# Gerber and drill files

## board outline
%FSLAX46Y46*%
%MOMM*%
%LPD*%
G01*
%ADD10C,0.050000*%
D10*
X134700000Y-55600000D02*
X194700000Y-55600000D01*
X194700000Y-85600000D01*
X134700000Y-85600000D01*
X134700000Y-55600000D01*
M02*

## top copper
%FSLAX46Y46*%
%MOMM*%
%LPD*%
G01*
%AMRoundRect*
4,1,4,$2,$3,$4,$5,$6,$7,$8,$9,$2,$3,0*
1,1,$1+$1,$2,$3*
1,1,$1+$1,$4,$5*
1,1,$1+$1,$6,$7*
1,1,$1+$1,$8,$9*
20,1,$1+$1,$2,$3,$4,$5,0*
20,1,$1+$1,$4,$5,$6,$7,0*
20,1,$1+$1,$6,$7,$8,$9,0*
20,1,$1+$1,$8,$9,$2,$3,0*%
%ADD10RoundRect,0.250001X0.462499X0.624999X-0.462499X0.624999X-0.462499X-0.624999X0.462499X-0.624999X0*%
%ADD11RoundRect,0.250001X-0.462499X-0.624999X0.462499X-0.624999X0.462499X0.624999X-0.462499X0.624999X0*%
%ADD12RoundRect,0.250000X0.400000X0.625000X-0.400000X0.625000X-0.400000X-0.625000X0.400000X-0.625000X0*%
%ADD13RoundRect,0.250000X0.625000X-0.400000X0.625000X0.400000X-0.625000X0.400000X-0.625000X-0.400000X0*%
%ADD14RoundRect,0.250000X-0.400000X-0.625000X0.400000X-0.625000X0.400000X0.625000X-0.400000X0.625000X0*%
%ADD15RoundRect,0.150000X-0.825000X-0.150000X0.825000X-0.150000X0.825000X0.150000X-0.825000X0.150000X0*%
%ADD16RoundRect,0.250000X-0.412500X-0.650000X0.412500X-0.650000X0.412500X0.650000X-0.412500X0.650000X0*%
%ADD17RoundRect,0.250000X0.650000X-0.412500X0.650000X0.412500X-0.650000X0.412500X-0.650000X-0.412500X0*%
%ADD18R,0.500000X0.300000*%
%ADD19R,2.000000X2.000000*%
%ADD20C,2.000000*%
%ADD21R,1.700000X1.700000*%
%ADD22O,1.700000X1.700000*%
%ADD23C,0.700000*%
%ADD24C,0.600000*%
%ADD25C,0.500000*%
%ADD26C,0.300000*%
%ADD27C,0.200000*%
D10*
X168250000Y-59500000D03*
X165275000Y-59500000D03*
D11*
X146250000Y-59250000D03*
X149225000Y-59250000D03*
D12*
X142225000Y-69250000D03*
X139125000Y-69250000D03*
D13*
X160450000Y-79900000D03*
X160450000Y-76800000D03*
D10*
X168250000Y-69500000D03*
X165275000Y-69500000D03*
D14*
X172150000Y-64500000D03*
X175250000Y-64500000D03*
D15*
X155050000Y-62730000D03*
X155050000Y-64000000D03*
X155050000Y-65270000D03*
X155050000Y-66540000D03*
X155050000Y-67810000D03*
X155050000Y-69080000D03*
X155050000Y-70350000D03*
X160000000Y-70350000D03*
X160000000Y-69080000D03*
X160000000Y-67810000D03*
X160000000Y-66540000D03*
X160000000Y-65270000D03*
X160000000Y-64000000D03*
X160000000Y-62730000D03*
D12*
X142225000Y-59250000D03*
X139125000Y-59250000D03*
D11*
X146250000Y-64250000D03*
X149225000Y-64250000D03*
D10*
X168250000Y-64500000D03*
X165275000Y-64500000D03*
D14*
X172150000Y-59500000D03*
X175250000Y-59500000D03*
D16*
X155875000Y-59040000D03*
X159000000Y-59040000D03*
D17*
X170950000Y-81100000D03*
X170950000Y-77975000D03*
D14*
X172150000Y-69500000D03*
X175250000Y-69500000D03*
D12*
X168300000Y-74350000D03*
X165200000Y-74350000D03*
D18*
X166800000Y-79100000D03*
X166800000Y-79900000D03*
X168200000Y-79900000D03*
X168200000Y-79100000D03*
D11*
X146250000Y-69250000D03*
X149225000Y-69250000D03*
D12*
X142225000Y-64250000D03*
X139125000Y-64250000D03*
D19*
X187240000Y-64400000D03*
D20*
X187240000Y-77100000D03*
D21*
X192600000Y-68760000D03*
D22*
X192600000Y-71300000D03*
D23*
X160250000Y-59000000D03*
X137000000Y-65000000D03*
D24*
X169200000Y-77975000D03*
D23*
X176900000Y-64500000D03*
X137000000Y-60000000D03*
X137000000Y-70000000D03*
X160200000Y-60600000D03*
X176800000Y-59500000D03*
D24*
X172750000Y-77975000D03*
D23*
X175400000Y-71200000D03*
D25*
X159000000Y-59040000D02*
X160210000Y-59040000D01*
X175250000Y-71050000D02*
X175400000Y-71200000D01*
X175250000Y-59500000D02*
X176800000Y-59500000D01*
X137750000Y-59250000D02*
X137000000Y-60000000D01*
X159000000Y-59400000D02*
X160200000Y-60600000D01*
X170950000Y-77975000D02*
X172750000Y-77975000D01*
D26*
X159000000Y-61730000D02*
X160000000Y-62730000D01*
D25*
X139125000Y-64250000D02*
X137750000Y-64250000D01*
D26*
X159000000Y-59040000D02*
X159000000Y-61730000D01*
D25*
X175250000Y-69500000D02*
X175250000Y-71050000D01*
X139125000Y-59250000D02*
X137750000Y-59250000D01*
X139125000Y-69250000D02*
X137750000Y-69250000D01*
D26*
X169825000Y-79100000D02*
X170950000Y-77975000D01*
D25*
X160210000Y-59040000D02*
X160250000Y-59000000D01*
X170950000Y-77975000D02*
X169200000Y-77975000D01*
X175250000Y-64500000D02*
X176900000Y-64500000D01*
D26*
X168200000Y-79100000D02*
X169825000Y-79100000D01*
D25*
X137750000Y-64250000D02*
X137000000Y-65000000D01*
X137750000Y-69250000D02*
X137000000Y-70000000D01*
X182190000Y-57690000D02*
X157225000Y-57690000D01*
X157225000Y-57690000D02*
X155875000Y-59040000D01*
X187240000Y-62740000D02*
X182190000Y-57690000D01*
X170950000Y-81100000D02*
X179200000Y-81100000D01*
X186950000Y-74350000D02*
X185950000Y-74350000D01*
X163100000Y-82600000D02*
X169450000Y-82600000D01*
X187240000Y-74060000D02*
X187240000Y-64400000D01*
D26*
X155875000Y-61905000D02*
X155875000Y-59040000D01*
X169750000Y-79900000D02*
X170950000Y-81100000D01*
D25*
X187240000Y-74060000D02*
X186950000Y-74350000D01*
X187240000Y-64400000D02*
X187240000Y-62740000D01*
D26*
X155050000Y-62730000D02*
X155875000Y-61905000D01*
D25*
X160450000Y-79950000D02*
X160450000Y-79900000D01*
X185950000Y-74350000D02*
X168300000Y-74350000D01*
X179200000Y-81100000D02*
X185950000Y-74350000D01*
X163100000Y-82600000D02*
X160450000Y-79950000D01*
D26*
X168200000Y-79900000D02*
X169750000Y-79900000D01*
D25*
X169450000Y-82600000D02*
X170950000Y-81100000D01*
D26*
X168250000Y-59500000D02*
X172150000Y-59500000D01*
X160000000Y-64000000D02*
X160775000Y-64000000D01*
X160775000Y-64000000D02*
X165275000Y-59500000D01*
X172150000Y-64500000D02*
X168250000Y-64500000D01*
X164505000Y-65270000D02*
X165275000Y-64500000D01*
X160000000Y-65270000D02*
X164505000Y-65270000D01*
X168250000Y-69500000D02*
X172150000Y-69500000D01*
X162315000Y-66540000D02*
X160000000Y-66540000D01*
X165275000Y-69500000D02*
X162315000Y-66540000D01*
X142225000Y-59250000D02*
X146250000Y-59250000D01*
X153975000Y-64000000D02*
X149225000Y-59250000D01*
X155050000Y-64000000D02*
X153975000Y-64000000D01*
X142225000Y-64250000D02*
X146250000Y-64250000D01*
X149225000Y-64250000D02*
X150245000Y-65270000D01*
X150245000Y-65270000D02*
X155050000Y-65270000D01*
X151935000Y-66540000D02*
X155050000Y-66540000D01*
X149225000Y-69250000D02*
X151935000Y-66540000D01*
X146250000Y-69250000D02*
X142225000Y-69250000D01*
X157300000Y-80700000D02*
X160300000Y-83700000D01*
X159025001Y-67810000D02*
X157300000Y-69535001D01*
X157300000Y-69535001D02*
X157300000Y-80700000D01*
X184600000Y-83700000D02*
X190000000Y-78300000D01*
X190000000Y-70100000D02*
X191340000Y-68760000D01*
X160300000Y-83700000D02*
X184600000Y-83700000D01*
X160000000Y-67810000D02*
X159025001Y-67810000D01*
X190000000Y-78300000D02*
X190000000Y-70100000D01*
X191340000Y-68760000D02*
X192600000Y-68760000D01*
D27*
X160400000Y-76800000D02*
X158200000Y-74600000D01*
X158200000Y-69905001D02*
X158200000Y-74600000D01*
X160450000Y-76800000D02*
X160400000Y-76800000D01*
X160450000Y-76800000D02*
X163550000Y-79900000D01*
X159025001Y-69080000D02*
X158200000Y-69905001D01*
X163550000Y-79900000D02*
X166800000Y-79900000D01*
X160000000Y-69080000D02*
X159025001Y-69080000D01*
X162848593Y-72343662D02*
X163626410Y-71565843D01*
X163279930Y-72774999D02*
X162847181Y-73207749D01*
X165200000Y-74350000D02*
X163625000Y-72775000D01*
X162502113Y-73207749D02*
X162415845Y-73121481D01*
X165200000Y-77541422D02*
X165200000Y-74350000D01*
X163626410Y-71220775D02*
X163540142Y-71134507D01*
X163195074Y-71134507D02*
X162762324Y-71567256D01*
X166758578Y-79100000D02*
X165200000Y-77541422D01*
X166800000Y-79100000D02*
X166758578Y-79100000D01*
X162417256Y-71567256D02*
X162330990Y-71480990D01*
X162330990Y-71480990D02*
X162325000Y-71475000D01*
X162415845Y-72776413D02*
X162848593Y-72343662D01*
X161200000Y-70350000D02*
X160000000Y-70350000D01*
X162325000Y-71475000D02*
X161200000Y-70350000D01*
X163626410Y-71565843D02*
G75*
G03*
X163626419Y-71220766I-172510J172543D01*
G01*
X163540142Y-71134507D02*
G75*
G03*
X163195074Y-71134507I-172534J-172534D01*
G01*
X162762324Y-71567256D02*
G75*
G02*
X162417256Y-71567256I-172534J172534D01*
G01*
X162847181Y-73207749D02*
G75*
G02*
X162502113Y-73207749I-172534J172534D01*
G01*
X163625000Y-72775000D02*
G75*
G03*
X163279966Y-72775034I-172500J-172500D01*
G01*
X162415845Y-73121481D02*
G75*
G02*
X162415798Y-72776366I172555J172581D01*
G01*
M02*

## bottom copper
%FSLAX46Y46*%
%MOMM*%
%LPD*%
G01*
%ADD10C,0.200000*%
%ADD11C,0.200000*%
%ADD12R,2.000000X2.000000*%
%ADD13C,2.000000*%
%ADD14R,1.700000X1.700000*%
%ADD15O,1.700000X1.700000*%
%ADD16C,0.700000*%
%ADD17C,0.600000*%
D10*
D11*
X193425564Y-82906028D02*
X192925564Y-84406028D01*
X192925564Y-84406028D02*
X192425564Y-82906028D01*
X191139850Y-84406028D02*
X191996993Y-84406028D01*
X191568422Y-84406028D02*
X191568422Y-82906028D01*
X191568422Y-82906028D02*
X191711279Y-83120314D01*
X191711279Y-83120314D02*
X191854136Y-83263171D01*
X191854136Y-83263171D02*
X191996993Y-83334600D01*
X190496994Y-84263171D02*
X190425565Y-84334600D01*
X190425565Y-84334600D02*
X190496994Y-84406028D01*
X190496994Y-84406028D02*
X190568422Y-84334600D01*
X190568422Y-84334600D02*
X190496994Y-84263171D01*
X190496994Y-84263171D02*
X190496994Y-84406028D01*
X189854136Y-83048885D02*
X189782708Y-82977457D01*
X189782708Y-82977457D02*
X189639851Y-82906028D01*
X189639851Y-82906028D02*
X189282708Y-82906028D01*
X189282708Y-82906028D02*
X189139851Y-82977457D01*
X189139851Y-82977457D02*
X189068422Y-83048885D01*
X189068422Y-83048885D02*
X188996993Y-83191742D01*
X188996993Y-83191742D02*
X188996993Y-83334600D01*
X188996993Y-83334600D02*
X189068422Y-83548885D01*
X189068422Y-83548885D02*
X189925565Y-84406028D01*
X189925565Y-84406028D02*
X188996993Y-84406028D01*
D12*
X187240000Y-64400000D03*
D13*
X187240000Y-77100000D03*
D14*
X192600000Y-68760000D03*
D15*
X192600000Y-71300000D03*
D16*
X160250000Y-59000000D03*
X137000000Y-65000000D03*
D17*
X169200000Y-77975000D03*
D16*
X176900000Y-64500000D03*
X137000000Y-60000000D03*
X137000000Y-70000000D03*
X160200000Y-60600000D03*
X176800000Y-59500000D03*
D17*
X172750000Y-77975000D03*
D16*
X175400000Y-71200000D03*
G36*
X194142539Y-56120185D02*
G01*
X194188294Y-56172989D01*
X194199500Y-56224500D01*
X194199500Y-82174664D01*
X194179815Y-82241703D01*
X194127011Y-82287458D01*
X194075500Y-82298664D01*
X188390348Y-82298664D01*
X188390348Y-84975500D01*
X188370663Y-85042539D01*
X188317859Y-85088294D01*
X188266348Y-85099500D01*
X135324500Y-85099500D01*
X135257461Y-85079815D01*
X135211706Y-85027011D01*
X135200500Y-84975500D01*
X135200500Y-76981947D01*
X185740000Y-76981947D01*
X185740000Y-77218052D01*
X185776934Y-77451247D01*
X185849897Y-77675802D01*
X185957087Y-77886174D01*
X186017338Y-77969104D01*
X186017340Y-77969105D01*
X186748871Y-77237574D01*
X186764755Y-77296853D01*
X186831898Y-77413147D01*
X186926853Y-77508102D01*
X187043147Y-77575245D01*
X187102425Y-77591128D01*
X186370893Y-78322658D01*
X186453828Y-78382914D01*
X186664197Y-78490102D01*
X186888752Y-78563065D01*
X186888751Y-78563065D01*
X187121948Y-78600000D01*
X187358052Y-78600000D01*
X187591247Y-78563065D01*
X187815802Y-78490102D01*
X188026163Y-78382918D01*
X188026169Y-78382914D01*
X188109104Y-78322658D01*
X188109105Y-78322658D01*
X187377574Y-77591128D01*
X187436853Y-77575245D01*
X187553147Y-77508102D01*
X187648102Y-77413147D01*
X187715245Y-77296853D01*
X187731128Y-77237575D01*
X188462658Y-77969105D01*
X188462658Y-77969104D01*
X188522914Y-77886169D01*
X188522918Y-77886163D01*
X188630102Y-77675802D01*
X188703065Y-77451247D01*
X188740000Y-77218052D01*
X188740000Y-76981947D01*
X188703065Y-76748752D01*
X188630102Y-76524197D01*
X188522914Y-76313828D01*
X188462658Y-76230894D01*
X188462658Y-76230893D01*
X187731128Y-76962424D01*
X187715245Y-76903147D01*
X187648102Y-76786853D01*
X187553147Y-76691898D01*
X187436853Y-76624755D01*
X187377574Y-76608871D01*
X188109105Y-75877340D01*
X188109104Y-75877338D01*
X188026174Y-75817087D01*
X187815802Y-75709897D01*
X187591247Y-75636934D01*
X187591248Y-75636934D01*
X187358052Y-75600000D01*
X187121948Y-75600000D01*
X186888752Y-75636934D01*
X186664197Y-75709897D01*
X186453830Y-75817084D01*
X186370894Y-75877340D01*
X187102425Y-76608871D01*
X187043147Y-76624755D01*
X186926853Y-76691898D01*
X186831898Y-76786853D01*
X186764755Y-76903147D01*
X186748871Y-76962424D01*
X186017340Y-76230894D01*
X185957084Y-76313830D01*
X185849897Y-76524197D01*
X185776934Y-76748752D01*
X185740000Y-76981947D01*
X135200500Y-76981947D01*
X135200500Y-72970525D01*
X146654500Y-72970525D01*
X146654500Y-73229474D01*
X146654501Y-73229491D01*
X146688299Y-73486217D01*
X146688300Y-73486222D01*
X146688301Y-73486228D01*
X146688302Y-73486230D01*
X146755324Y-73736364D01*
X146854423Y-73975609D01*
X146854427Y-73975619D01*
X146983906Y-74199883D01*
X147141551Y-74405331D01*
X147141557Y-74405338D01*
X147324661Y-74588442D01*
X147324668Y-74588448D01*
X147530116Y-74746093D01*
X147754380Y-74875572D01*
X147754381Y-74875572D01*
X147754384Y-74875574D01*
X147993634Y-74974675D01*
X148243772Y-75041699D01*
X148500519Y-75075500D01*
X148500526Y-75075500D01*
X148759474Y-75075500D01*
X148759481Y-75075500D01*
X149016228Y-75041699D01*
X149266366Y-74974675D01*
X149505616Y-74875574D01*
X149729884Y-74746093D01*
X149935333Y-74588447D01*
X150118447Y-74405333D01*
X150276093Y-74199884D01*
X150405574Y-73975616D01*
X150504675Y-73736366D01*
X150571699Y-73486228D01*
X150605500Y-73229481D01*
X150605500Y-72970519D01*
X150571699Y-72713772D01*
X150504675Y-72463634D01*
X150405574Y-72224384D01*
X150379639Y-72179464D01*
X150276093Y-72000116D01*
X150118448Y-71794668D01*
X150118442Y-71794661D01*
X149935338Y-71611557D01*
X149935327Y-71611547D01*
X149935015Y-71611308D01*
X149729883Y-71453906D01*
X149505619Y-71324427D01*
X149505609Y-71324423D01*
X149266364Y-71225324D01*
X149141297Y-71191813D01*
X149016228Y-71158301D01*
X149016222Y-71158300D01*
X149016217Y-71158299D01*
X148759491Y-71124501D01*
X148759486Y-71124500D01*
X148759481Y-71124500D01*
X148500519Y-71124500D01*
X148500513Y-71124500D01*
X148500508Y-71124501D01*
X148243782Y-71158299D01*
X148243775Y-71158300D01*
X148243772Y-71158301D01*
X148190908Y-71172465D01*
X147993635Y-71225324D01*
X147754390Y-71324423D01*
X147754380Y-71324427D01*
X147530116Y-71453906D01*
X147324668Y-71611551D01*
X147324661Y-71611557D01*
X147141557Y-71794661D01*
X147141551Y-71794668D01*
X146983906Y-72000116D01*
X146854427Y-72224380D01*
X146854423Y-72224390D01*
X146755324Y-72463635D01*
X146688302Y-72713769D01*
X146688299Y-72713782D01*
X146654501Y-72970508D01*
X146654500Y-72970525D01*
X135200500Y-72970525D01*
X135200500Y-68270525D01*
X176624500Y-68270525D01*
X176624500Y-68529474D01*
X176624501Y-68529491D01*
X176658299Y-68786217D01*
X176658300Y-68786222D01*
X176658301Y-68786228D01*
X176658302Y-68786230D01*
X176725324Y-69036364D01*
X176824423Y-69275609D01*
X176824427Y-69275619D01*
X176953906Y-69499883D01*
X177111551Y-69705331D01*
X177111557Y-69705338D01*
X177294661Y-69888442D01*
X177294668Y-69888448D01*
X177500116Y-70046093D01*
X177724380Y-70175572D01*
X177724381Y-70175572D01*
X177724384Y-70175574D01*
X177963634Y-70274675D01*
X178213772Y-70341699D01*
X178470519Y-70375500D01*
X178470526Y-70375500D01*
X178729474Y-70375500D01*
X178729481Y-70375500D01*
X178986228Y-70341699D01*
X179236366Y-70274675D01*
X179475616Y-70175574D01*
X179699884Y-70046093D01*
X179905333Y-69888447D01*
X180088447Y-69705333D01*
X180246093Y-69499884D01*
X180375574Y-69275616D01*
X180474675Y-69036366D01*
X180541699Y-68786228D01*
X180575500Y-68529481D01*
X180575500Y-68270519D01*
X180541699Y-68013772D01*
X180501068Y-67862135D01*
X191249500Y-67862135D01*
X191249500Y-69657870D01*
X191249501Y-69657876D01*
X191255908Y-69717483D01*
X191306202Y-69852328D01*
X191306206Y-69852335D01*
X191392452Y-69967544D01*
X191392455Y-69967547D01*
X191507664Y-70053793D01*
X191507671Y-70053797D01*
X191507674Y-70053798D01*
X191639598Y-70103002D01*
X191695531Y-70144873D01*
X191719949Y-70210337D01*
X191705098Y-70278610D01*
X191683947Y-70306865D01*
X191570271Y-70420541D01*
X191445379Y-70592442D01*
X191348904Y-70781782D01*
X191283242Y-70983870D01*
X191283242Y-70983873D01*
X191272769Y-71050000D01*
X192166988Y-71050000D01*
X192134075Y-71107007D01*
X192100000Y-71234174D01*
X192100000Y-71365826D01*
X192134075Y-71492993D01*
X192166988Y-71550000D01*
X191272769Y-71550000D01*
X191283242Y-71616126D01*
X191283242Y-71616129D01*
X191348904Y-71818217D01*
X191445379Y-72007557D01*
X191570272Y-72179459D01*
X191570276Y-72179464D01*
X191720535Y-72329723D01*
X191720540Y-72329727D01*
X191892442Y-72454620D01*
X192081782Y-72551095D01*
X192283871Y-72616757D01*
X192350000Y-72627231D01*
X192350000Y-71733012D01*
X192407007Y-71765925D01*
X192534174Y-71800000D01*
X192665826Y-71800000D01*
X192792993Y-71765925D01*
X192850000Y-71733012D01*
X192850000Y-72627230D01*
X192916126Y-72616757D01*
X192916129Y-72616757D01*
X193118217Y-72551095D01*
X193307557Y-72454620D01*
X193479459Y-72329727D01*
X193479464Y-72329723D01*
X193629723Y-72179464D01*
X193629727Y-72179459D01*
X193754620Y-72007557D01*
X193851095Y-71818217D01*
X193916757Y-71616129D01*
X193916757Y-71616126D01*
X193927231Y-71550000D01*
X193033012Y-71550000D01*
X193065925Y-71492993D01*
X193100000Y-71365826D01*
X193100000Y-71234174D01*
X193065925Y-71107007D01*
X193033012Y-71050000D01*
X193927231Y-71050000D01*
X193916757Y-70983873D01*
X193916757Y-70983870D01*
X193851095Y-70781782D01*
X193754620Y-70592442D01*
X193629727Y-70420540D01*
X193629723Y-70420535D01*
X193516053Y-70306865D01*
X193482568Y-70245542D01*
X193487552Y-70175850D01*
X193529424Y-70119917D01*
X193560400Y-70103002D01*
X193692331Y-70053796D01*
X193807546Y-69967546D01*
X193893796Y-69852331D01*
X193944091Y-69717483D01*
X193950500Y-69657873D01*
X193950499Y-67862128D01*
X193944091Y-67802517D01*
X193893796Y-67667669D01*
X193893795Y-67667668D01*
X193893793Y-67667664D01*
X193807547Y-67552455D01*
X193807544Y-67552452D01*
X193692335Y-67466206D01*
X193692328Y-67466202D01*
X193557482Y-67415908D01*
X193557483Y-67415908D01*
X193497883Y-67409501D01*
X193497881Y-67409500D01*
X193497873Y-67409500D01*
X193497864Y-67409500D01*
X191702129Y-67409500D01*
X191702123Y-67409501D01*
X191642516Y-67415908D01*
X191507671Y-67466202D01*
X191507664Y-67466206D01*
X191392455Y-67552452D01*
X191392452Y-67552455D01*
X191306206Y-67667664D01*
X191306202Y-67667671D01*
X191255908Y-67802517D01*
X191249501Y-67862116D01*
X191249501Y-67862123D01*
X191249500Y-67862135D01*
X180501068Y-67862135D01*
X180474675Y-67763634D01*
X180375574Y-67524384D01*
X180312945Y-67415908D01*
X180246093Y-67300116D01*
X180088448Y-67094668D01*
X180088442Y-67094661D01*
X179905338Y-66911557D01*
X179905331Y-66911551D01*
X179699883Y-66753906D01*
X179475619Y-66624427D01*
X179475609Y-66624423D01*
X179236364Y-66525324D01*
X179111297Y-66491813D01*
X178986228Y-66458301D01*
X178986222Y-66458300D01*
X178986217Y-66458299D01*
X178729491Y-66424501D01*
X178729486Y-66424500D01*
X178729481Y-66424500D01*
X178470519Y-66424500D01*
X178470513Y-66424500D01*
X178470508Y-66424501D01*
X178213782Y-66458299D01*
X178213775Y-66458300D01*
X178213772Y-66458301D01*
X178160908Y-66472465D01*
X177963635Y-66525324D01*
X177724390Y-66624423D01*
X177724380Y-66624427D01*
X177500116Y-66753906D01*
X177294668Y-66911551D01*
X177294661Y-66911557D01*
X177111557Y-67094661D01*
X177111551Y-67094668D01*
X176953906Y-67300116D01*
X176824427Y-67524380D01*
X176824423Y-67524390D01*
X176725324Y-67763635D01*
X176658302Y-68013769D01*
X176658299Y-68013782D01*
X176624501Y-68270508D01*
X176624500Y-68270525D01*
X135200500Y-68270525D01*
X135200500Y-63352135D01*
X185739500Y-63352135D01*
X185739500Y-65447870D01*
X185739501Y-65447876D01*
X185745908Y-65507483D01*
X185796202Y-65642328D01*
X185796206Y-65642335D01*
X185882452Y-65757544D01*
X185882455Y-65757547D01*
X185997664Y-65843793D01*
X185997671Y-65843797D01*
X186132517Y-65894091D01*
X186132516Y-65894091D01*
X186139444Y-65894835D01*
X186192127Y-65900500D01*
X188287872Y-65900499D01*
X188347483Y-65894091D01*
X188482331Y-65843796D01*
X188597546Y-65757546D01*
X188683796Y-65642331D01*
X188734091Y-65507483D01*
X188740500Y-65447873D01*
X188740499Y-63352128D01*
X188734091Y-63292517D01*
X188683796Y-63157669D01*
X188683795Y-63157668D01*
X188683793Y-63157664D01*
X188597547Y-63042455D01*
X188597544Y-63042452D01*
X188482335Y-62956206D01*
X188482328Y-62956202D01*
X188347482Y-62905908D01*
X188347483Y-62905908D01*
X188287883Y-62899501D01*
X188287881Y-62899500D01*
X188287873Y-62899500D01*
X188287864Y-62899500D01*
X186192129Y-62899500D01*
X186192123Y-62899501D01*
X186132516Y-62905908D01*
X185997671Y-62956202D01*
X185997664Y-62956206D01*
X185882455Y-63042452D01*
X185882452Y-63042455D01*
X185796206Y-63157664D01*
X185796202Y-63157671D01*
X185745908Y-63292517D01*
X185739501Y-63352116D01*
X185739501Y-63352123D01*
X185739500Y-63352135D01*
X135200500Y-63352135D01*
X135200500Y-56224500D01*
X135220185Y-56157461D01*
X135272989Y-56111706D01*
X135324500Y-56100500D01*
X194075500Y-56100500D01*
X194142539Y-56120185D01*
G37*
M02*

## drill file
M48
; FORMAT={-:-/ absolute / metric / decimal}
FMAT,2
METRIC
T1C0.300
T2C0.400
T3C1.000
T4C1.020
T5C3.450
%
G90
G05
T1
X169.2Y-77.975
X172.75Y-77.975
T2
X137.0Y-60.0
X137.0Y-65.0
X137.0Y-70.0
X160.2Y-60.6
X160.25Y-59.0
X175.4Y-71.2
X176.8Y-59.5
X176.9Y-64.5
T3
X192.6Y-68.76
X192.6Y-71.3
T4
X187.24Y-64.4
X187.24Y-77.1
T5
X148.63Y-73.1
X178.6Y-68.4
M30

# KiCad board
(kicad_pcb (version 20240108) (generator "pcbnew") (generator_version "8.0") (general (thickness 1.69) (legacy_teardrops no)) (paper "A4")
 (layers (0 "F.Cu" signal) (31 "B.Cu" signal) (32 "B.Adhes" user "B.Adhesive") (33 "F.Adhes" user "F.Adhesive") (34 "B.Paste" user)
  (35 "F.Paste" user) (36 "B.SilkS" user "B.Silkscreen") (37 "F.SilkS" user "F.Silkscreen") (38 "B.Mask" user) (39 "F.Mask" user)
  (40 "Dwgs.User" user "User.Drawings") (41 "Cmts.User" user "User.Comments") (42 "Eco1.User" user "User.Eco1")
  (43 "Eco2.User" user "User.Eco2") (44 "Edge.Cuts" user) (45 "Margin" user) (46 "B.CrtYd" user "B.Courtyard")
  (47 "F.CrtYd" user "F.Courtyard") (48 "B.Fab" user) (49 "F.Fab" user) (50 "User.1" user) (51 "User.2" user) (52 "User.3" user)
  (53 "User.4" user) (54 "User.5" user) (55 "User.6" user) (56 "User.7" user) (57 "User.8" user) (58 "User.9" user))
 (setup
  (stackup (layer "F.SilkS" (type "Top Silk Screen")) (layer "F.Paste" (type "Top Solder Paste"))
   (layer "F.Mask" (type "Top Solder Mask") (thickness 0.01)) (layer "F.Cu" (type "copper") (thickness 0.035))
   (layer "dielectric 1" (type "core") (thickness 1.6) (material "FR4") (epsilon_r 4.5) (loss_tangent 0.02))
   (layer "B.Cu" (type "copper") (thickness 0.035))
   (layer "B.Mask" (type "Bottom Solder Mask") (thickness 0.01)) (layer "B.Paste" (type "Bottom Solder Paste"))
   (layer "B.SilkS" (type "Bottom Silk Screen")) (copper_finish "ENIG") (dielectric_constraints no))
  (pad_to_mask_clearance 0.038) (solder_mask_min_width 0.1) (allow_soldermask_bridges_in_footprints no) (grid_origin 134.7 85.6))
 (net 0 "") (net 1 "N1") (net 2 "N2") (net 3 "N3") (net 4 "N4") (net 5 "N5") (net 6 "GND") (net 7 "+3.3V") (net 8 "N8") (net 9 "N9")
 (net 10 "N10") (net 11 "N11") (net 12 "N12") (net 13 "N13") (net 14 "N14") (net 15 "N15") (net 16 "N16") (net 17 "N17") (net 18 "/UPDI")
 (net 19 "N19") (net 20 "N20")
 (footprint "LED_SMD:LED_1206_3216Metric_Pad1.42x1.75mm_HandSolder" (layer "F.Cu") (at 166.7625 59.5 180)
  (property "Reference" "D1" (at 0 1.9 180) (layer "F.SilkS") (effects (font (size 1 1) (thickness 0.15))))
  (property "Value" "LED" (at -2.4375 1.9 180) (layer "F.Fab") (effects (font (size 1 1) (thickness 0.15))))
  (pad "1" smd roundrect (at -1.4875 0 180) (size 1.425 1.75) (layers "F.Cu" "F.Paste" "F.Mask") (roundrect_rratio 0.175439) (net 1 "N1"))
  (pad "2" smd roundrect (at 1.4875 0 180) (size 1.425 1.75) (layers "F.Cu" "F.Paste" "F.Mask") (roundrect_rratio 0.175439) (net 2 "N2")))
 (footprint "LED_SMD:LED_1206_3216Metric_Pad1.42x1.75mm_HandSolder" (layer "F.Cu") (at 147.7375 59.25)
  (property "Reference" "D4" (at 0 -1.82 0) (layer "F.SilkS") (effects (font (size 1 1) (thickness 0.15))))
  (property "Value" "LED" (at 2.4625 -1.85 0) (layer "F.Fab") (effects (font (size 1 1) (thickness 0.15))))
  (pad "1" smd roundrect (at -1.4875 0) (size 1.425 1.75) (layers "F.Cu" "F.Paste" "F.Mask") (roundrect_rratio 0.175439) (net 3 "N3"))
  (pad "2" smd roundrect (at 1.4875 0) (size 1.425 1.75) (layers "F.Cu" "F.Paste" "F.Mask") (roundrect_rratio 0.175439) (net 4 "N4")))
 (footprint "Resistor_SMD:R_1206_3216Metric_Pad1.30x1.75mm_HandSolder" (layer "F.Cu") (at 140.675 69.25 180)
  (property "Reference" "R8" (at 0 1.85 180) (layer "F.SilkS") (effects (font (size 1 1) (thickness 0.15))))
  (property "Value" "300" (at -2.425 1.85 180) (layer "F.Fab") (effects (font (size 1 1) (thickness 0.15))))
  (pad "1" smd roundrect (at -1.55 0 180) (size 1.3 1.75) (layers "F.Cu" "F.Paste" "F.Mask") (roundrect_rratio 0.192308) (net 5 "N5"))
  (pad "2" smd roundrect (at 1.55 0 180) (size 1.3 1.75) (layers "F.Cu" "F.Paste" "F.Mask") (roundrect_rratio 0.192308) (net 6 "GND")))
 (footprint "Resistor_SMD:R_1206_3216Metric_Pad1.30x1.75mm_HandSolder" (layer "F.Cu") (at 160.45 78.35 90)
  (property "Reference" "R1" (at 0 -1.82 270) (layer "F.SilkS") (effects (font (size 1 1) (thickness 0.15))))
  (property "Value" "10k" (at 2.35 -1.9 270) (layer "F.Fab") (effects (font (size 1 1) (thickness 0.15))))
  (pad "1" smd roundrect (at -1.55 0 90) (size 1.3 1.75) (layers "F.Cu" "F.Paste" "F.Mask") (roundrect_rratio 0.192308) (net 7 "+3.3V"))
  (pad "2" smd roundrect (at 1.55 0 90) (size 1.3 1.75) (layers "F.Cu" "F.Paste" "F.Mask") (roundrect_rratio 0.192308) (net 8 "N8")))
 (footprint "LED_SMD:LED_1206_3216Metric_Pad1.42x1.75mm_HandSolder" (layer "F.Cu") (at 166.7625 69.5 180)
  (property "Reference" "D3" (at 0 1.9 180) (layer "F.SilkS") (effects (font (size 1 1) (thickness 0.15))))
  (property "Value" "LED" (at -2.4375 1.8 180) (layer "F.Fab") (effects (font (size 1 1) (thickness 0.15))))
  (pad "1" smd roundrect (at -1.4875 0 180) (size 1.425 1.75) (layers "F.Cu" "F.Paste" "F.Mask") (roundrect_rratio 0.175439) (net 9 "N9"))
  (pad "2" smd roundrect (at 1.4875 0 180) (size 1.425 1.75) (layers "F.Cu" "F.Paste" "F.Mask") (roundrect_rratio 0.175439) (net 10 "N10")))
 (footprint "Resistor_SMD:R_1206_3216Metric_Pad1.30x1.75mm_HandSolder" (layer "F.Cu") (at 173.7 64.5)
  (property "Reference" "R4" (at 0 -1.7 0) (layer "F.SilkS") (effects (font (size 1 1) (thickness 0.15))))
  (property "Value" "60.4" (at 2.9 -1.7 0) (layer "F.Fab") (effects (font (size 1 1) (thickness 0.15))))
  (pad "1" smd roundrect (at -1.55 0) (size 1.3 1.75) (layers "F.Cu" "F.Paste" "F.Mask") (roundrect_rratio 0.192308) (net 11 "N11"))
  (pad "2" smd roundrect (at 1.55 0) (size 1.3 1.75) (layers "F.Cu" "F.Paste" "F.Mask") (roundrect_rratio 0.192308) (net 6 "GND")))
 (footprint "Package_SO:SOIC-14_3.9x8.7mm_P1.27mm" (layer "F.Cu") (at 157.525 66.54)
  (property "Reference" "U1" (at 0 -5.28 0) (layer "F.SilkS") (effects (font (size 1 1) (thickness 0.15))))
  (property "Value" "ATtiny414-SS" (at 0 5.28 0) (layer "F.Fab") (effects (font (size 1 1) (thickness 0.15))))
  (pad "1" smd roundrect (at -2.475 -3.81) (size 1.95 0.6) (layers "F.Cu" "F.Paste" "F.Mask") (roundrect_rratio 0.25) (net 7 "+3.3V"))
  (pad "2" smd roundrect (at -2.475 -2.54) (size 1.95 0.6) (layers "F.Cu" "F.Paste" "F.Mask") (roundrect_rratio 0.25) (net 4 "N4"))
  (pad "3" smd roundrect (at -2.475 -1.27) (size 1.95 0.6) (layers "F.Cu" "F.Paste" "F.Mask") (roundrect_rratio 0.25) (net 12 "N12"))
  (pad "4" smd roundrect (at -2.475 0) (size 1.95 0.6) (layers "F.Cu" "F.Paste" "F.Mask") (roundrect_rratio 0.25) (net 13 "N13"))
  (pad "5" smd roundrect (at -2.475 1.27) (size 1.95 0.6) (layers "F.Cu" "F.Paste" "F.Mask") (roundrect_rratio 0.25) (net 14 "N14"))
  (pad "6" smd roundrect (at -2.475 2.54) (size 1.95 0.6) (layers "F.Cu" "F.Paste" "F.Mask") (roundrect_rratio 0.25) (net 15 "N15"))
  (pad "7" smd roundrect (at -2.475 3.81) (size 1.95 0.6) (layers "F.Cu" "F.Paste" "F.Mask") (roundrect_rratio 0.25) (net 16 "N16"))
  (pad "8" smd roundrect (at 2.475 3.81) (size 1.95 0.6) (layers "F.Cu" "F.Paste" "F.Mask") (roundrect_rratio 0.25) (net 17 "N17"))
  (pad "9" smd roundrect (at 2.475 2.54) (size 1.95 0.6) (layers "F.Cu" "F.Paste" "F.Mask") (roundrect_rratio 0.25) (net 8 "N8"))
  (pad "10" smd roundrect (at 2.475 1.27) (size 1.95 0.6) (layers "F.Cu" "F.Paste" "F.Mask") (roundrect_rratio 0.25) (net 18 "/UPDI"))
  (pad "11" smd roundrect (at 2.475 0) (size 1.95 0.6) (layers "F.Cu" "F.Paste" "F.Mask") (roundrect_rratio 0.25) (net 10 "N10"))
  (pad "12" smd roundrect (at 2.475 -1.27) (size 1.95 0.6) (layers "F.Cu" "F.Paste" "F.Mask") (roundrect_rratio 0.25) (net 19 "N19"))
  (pad "13" smd roundrect (at 2.475 -2.54) (size 1.95 0.6) (layers "F.Cu" "F.Paste" "F.Mask") (roundrect_rratio 0.25) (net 2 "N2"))
  (pad "14" smd roundrect (at 2.475 -3.81) (size 1.95 0.6) (layers "F.Cu" "F.Paste" "F.Mask") (roundrect_rratio 0.25) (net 6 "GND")))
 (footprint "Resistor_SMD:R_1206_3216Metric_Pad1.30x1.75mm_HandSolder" (layer "F.Cu") (at 140.675 59.25 180)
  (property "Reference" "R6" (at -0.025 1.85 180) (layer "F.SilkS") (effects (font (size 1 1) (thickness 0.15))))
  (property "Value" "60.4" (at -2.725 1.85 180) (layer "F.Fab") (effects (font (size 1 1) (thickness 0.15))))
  (pad "1" smd roundrect (at -1.55 0 180) (size 1.3 1.75) (layers "F.Cu" "F.Paste" "F.Mask") (roundrect_rratio 0.192308) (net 3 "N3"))
  (pad "2" smd roundrect (at 1.55 0 180) (size 1.3 1.75) (layers "F.Cu" "F.Paste" "F.Mask") (roundrect_rratio 0.192308) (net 6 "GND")))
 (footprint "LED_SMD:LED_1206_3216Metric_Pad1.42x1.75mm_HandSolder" (layer "F.Cu") (at 147.7375 64.25)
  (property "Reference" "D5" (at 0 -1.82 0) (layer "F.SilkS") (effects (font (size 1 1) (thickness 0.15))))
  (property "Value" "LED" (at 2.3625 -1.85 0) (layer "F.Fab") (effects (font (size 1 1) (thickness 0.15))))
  (pad "1" smd roundrect (at -1.4875 0) (size 1.425 1.75) (layers "F.Cu" "F.Paste" "F.Mask") (roundrect_rratio 0.175439) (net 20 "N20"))
  (pad "2" smd roundrect (at 1.4875 0) (size 1.425 1.75) (layers "F.Cu" "F.Paste" "F.Mask") (roundrect_rratio 0.175439) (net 12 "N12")))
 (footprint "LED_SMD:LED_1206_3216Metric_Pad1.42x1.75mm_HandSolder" (layer "F.Cu") (at 166.7625 64.5 180)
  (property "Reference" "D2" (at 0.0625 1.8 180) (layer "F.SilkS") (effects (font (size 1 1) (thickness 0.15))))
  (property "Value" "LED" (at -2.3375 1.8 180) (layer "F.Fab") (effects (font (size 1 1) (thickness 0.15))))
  (pad "1" smd roundrect (at -1.4875 0 180) (size 1.425 1.75) (layers "F.Cu" "F.Paste" "F.Mask") (roundrect_rratio 0.175439) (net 11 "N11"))
  (pad "2" smd roundrect (at 1.4875 0 180) (size 1.425 1.75) (layers "F.Cu" "F.Paste" "F.Mask") (roundrect_rratio 0.175439) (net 19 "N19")))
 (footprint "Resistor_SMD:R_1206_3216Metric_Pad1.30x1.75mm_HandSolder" (layer "F.Cu") (at 173.7 59.5)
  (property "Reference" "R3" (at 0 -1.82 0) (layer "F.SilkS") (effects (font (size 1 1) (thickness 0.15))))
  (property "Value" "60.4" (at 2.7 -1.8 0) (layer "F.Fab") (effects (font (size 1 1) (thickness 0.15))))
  (pad "1" smd roundrect (at -1.55 0) (size 1.3 1.75) (layers "F.Cu" "F.Paste" "F.Mask") (roundrect_rratio 0.192308) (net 1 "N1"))
  (pad "2" smd roundrect (at 1.55 0) (size 1.3 1.75) (layers "F.Cu" "F.Paste" "F.Mask") (roundrect_rratio 0.192308) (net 6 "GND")))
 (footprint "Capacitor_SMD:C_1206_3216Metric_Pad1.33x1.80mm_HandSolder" (layer "F.Cu") (at 157.4375 59.04)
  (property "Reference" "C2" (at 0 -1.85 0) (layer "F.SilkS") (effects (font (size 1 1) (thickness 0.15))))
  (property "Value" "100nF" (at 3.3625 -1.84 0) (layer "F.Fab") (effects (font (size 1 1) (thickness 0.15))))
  (pad "1" smd roundrect (at -1.5625 0) (size 1.325 1.8) (layers "F.Cu" "F.Paste" "F.Mask") (roundrect_rratio 0.188679) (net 7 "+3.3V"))
  (pad "2" smd roundrect (at 1.5625 0) (size 1.325 1.8) (layers "F.Cu" "F.Paste" "F.Mask") (roundrect_rratio 0.188679) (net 6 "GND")))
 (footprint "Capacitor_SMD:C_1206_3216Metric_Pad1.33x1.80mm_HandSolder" (layer "F.Cu") (at 170.95 79.5375 90)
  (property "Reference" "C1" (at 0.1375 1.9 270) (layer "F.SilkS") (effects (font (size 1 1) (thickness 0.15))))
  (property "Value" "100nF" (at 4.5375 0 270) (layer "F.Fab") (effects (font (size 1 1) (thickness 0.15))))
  (pad "1" smd roundrect (at -1.5625 0 90) (size 1.325 1.8) (layers "F.Cu" "F.Paste" "F.Mask") (roundrect_rratio 0.188679) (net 7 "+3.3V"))
  (pad "2" smd roundrect (at 1.5625 0 90) (size 1.325 1.8) (layers "F.Cu" "F.Paste" "F.Mask") (roundrect_rratio 0.188679) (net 6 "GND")))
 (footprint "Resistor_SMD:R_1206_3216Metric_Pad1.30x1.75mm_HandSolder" (layer "F.Cu") (at 173.7 69.5)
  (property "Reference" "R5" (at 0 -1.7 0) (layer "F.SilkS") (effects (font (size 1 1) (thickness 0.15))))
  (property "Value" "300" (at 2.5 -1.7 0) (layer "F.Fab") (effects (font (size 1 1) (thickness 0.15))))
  (pad "1" smd roundrect (at -1.55 0) (size 1.3 1.75) (layers "F.Cu" "F.Paste" "F.Mask") (roundrect_rratio 0.192308) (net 9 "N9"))
  (pad "2" smd roundrect (at 1.55 0) (size 1.3 1.75) (layers "F.Cu" "F.Paste" "F.Mask") (roundrect_rratio 0.192308) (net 6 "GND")))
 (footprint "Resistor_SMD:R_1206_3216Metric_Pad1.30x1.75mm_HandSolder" (layer "F.Cu") (at 166.75 74.35 180)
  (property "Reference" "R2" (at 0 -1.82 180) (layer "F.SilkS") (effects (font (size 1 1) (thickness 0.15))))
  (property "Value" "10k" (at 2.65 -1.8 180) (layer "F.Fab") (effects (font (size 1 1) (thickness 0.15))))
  (pad "1" smd roundrect (at -1.55 0 180) (size 1.3 1.75) (layers "F.Cu" "F.Paste" "F.Mask") (roundrect_rratio 0.192308) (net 7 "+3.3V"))
  (pad "2" smd roundrect (at 1.55 0 180) (size 1.3 1.75) (layers "F.Cu" "F.Paste" "F.Mask") (roundrect_rratio 0.192308) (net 17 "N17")))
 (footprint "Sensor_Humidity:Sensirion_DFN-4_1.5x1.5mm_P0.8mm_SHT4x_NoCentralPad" (layer "F.Cu") (at 167.5 79.5)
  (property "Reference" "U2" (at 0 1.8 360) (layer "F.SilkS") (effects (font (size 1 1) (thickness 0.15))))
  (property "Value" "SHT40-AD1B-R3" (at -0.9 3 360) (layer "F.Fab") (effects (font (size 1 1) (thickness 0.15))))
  (pad "1" smd rect (at -0.7 -0.4) (size 0.5 0.3) (layers "F.Cu" "F.Paste" "F.Mask") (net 17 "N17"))
  (pad "2" smd rect (at -0.7 0.4) (size 0.5 0.3) (layers "F.Cu" "F.Paste" "F.Mask") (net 8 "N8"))
  (pad "3" smd rect (at 0.7 0.4) (size 0.5 0.3) (layers "F.Cu" "F.Paste" "F.Mask") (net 7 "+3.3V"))
  (pad "4" smd rect (at 0.7 -0.4) (size 0.5 0.3) (layers "F.Cu" "F.Paste" "F.Mask") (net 6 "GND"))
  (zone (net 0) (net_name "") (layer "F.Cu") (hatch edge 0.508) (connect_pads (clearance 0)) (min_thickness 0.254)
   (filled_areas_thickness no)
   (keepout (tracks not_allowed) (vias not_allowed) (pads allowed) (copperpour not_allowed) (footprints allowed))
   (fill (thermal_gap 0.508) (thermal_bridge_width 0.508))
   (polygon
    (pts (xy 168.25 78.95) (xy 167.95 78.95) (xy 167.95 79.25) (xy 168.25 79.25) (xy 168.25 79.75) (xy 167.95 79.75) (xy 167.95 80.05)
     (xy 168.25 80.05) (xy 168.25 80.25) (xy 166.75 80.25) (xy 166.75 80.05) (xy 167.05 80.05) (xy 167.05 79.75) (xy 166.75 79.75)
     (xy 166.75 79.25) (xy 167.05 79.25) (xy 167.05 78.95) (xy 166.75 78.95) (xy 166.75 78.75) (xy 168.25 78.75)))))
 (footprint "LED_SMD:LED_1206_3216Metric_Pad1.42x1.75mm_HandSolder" (layer "F.Cu") (at 147.7375 69.25)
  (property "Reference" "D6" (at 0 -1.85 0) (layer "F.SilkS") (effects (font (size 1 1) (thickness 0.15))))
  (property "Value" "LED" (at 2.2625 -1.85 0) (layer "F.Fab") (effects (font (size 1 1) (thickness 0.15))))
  (pad "1" smd roundrect (at -1.4875 0) (size 1.425 1.75) (layers "F.Cu" "F.Paste" "F.Mask") (roundrect_rratio 0.175439) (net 5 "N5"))
  (pad "2" smd roundrect (at 1.4875 0) (size 1.425 1.75) (layers "F.Cu" "F.Paste" "F.Mask") (roundrect_rratio 0.175439) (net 13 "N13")))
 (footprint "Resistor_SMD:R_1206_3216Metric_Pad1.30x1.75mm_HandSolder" (layer "F.Cu") (at 140.675 64.25 180)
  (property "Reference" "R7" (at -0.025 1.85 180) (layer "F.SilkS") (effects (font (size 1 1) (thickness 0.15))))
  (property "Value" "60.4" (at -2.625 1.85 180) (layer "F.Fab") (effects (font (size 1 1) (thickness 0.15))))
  (pad "1" smd roundrect (at -1.55 0 180) (size 1.3 1.75) (layers "F.Cu" "F.Paste" "F.Mask") (roundrect_rratio 0.192308) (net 20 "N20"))
  (pad "2" smd roundrect (at 1.55 0 180) (size 1.3 1.75) (layers "F.Cu" "F.Paste" "F.Mask") (roundrect_rratio 0.192308) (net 6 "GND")))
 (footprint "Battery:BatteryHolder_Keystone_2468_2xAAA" (layer "B.Cu") (at 187.24 64.4 180)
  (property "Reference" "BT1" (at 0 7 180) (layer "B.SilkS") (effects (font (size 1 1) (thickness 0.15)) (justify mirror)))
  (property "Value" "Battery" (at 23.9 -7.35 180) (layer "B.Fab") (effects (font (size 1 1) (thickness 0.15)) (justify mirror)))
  (pad "" np_thru_hole circle (at 8.64 -4 180) (size 3.45 3.45) (drill 3.45) (layers "*.Cu"))
  (pad "" np_thru_hole circle (at 38.61 -8.7 180) (size 3.45 3.45) (drill 3.45) (layers "*.Cu" "*.Mask"))
  (pad "1" thru_hole rect (at 0 0 180) (size 2 2) (drill 1.02) (layers "*.Cu" "*.Mask") (remove_unused_layers no) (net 7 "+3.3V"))
  (pad "2" thru_hole circle (at 0 -12.7 180) (size 2 2) (drill 1.02) (layers "*.Cu" "*.Mask") (remove_unused_layers no) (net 6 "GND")))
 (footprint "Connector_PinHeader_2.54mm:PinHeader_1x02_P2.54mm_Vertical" (layer "B.Cu") (at 192.6 68.76 180)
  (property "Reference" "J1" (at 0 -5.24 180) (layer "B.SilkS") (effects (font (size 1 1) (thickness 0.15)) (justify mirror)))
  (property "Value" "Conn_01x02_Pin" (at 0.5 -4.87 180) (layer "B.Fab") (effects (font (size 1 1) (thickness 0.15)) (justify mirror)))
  (pad "1" thru_hole rect (at 0 0 180) (size 1.7 1.7) (drill 1) (layers "*.Cu" "*.Mask") (remove_unused_layers no) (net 18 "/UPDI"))
  (pad "2" thru_hole oval (at 0 -2.54 180) (size 1.7 1.7) (drill 1) (layers "*.Cu" "*.Mask") (remove_unused_layers no) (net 6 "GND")))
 (gr_rect (start 134.7 55.6) (end 194.7 85.6) (stroke (width 0.05) (type default)) (fill none) (layer "Edge.Cuts"))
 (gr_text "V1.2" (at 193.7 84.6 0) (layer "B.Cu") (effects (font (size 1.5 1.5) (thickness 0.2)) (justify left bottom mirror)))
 (segment (start 159 59.04) (end 160.21 59.04) (width 0.5) (layer "F.Cu") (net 6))
 (segment (start 175.25 71.05) (end 175.4 71.2) (width 0.5) (layer "F.Cu") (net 6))
 (segment (start 175.25 59.5) (end 176.8 59.5) (width 0.5) (layer "F.Cu") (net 6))
 (segment (start 137.75 59.25) (end 137 60) (width 0.5) (layer "F.Cu") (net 6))
 (segment (start 159 59.4) (end 160.2 60.6) (width 0.5) (layer "F.Cu") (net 6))
 (segment (start 170.95 77.975) (end 172.75 77.975) (width 0.5) (layer "F.Cu") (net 6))
 (segment (start 159 61.73) (end 160 62.73) (width 0.3) (layer "F.Cu") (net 6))
 (segment (start 139.125 64.25) (end 137.75 64.25) (width 0.5) (layer "F.Cu") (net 6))
 (segment (start 159 59.04) (end 159 61.73) (width 0.3) (layer "F.Cu") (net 6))
 (segment (start 175.25 69.5) (end 175.25 71.05) (width 0.5) (layer "F.Cu") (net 6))
 (segment (start 139.125 59.25) (end 137.75 59.25) (width 0.5) (layer "F.Cu") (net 6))
 (segment (start 139.125 69.25) (end 137.75 69.25) (width 0.5) (layer "F.Cu") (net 6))
 (segment (start 169.825 79.1) (end 170.95 77.975) (width 0.3) (layer "F.Cu") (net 6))
 (segment (start 160.21 59.04) (end 160.25 59) (width 0.5) (layer "F.Cu") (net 6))
 (segment (start 170.95 77.975) (end 169.2 77.975) (width 0.5) (layer "F.Cu") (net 6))
 (segment (start 175.25 64.5) (end 176.9 64.5) (width 0.5) (layer "F.Cu") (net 6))
 (segment (start 168.2 79.1) (end 169.825 79.1) (width 0.3) (layer "F.Cu") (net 6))
 (segment (start 137.75 64.25) (end 137 65) (width 0.5) (layer "F.Cu") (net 6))
 (segment (start 137.75 69.25) (end 137 70) (width 0.5) (layer "F.Cu") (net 6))
 (via (at 160.25 59) (size 0.7) (drill 0.4) (layers "F.Cu" "B.Cu") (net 6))
 (via (at 137 65) (size 0.7) (drill 0.4) (layers "F.Cu" "B.Cu") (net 6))
 (via (at 169.2 77.975) (size 0.6) (drill 0.3) (layers "F.Cu" "B.Cu") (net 6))
 (via (at 176.9 64.5) (size 0.7) (drill 0.4) (layers "F.Cu" "B.Cu") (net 6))
 (via (at 137 60) (size 0.7) (drill 0.4) (layers "F.Cu" "B.Cu") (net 6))
 (via (at 137 70) (size 0.7) (drill 0.4) (layers "F.Cu" "B.Cu") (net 6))
 (via (at 160.2 60.6) (size 0.7) (drill 0.4) (layers "F.Cu" "B.Cu") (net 6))
 (via (at 176.8 59.5) (size 0.7) (drill 0.4) (layers "F.Cu" "B.Cu") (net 6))
 (via (at 172.75 77.975) (size 0.6) (drill 0.3) (layers "F.Cu" "B.Cu") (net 6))
 (via (at 175.4 71.2) (size 0.7) (drill 0.4) (layers "F.Cu" "B.Cu") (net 6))
 (segment (start 182.19 57.69) (end 157.225 57.69) (width 0.5) (layer "F.Cu") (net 7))
 (segment (start 157.225 57.69) (end 155.875 59.04) (width 0.5) (layer "F.Cu") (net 7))
 (segment (start 187.24 62.74) (end 182.19 57.69) (width 0.5) (layer "F.Cu") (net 7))
 (segment (start 170.95 81.1) (end 179.2 81.1) (width 0.5) (layer "F.Cu") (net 7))
 (segment (start 186.95 74.35) (end 185.95 74.35) (width 0.5) (layer "F.Cu") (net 7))
 (segment (start 163.1 82.6) (end 169.45 82.6) (width 0.5) (layer "F.Cu") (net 7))
 (segment (start 187.24 74.06) (end 187.24 64.4) (width 0.5) (layer "F.Cu") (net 7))
 (segment (start 155.875 61.905) (end 155.875 59.04) (width 0.3) (layer "F.Cu") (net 7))
 (segment (start 169.75 79.9) (end 170.95 81.1) (width 0.3) (layer "F.Cu") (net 7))
 (segment (start 187.24 74.06) (end 186.95 74.35) (width 0.5) (layer "F.Cu") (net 7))
 (segment (start 187.24 64.4) (end 187.24 62.74) (width 0.5) (layer "F.Cu") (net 7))
 (segment (start 155.05 62.73) (end 155.875 61.905) (width 0.3) (layer "F.Cu") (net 7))
 (segment (start 160.45 79.95) (end 160.45 79.9) (width 0.5) (layer "F.Cu") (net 7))
 (segment (start 185.95 74.35) (end 168.3 74.35) (width 0.5) (layer "F.Cu") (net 7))
 (segment (start 179.2 81.1) (end 185.95 74.35) (width 0.5) (layer "F.Cu") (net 7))
 (segment (start 163.1 82.6) (end 160.45 79.95) (width 0.5) (layer "F.Cu") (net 7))
 (segment (start 168.2 79.9) (end 169.75 79.9) (width 0.3) (layer "F.Cu") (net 7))
 (segment (start 169.45 82.6) (end 170.95 81.1) (width 0.5) (layer "F.Cu") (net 7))
 (segment (start 168.25 59.5) (end 172.15 59.5) (width 0.3) (layer "F.Cu") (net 1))
 (segment (start 160 64) (end 160.775 64) (width 0.3) (layer "F.Cu") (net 2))
 (segment (start 160.775 64) (end 165.275 59.5) (width 0.3) (layer "F.Cu") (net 2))
 (segment (start 172.15 64.5) (end 168.25 64.5) (width 0.3) (layer "F.Cu") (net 11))
 (segment (start 164.505 65.27) (end 165.275 64.5) (width 0.3) (layer "F.Cu") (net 19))
 (segment (start 160 65.27) (end 164.505 65.27) (width 0.3) (layer "F.Cu") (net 19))
 (segment (start 168.25 69.5) (end 172.15 69.5) (width 0.3) (layer "F.Cu") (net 9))
 (segment (start 162.315 66.54) (end 160 66.54) (width 0.3) (layer "F.Cu") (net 10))
 (segment (start 165.275 69.5) (end 162.315 66.54) (width 0.3) (layer "F.Cu") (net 10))
 (segment (start 142.225 59.25) (end 146.25 59.25) (width 0.3) (layer "F.Cu") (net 3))
 (segment (start 153.975 64) (end 149.225 59.25) (width 0.3) (layer "F.Cu") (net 4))
 (segment (start 155.05 64) (end 153.975 64) (width 0.3) (layer "F.Cu") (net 4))
 (segment (start 142.225 64.25) (end 146.25 64.25) (width 0.3) (layer "F.Cu") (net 20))
 (segment (start 149.225 64.25) (end 150.245 65.27) (width 0.3) (layer "F.Cu") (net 12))
 (segment (start 150.245 65.27) (end 155.05 65.27) (width 0.3) (layer "F.Cu") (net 12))
 (segment (start 151.935 66.54) (end 155.05 66.54) (width 0.3) (layer "F.Cu") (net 13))
 (segment (start 149.225 69.25) (end 151.935 66.54) (width 0.3) (layer "F.Cu") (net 13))
 (segment (start 146.25 69.25) (end 142.225 69.25) (width 0.3) (layer "F.Cu") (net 5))
 (segment (start 157.3 80.7) (end 160.3 83.7) (width 0.3) (layer "F.Cu") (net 18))
 (segment (start 159.025001 67.81) (end 157.3 69.535001) (width 0.3) (layer "F.Cu") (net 18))
 (segment (start 157.3 69.535001) (end 157.3 80.7) (width 0.3) (layer "F.Cu") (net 18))
 (segment (start 184.6 83.7) (end 190 78.3) (width 0.3) (layer "F.Cu") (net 18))
 (segment (start 190 70.1) (end 191.34 68.76) (width 0.3) (layer "F.Cu") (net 18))
 (segment (start 160.3 83.7) (end 184.6 83.7) (width 0.3) (layer "F.Cu") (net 18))
 (segment (start 160 67.81) (end 159.025001 67.81) (width 0.3) (layer "F.Cu") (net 18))
 (segment (start 190 78.3) (end 190 70.1) (width 0.3) (layer "F.Cu") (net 18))
 (segment (start 191.34 68.76) (end 192.6 68.76) (width 0.3) (layer "F.Cu") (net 18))
 (segment (start 160.4 76.8) (end 158.2 74.6) (width 0.2) (layer "F.Cu") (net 8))
 (segment (start 158.2 69.905001) (end 158.2 74.6) (width 0.2) (layer "F.Cu") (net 8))
 (segment (start 160.45 76.8) (end 160.4 76.8) (width 0.2) (layer "F.Cu") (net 8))
 (segment (start 160.45 76.8) (end 163.55 79.9) (width 0.2) (layer "F.Cu") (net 8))
 (segment (start 159.025001 69.08) (end 158.2 69.905001) (width 0.2) (layer "F.Cu") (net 8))
 (segment (start 163.55 79.9) (end 166.8 79.9) (width 0.2) (layer "F.Cu") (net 8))
 (segment (start 160 69.08) (end 159.025001 69.08) (width 0.2) (layer "F.Cu") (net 8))
 (segment (start 162.848593 72.343662) (end 163.62641 71.565843) (width 0.2) (layer "F.Cu") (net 17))
 (segment (start 163.27993 72.774999) (end 162.847181 73.207749) (width 0.2) (layer "F.Cu") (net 17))
 (segment (start 165.2 74.35) (end 163.625 72.775) (width 0.2) (layer "F.Cu") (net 17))
 (segment (start 162.502113 73.207749) (end 162.415845 73.121481) (width 0.2) (layer "F.Cu") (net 17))
 (segment (start 165.2 77.541422) (end 165.2 74.35) (width 0.2) (layer "F.Cu") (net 17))
 (segment (start 163.62641 71.220775) (end 163.540142 71.134507) (width 0.2) (layer "F.Cu") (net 17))
 (segment (start 163.195074 71.134507) (end 162.762324 71.567256) (width 0.2) (layer "F.Cu") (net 17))
 (segment (start 166.758578 79.1) (end 165.2 77.541422) (width 0.2) (layer "F.Cu") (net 17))
 (segment (start 166.8 79.1) (end 166.758578 79.1) (width 0.2) (layer "F.Cu") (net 17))
 (segment (start 162.417256 71.567256) (end 162.33099 71.48099) (width 0.2) (layer "F.Cu") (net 17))
 (segment (start 162.33099 71.48099) (end 162.325 71.475) (width 0.2) (layer "F.Cu") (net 17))
 (segment (start 162.415845 72.776413) (end 162.848593 72.343662) (width 0.2) (layer "F.Cu") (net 17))
 (segment (start 161.2 70.35) (end 160 70.35) (width 0.2) (layer "F.Cu") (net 17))
 (segment (start 162.325 71.475) (end 161.2 70.35) (width 0.2) (layer "F.Cu") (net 17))
 (arc (start 163.62641 71.565843) (mid 163.697876 71.393309) (end 163.62641 71.220775) (width 0.2) (layer "F.Cu") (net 17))
 (arc (start 163.540142 71.134507) (mid 163.367608 71.063041) (end 163.195074 71.134507) (width 0.2) (layer "F.Cu") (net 17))
 (arc (start 162.762324 71.567256) (mid 162.58979 71.638722) (end 162.417256 71.567256) (width 0.2) (layer "F.Cu") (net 17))
 (arc (start 162.847181 73.207749) (mid 162.674647 73.279215) (end 162.502113 73.207749) (width 0.2) (layer "F.Cu") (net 17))
 (arc (start 163.625 72.775) (mid 163.452465 72.703532) (end 163.27993 72.774999) (width 0.2) (layer "F.Cu") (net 17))
 (arc (start 162.415845 73.121481) (mid 162.344379 72.948947) (end 162.415845 72.776413) (width 0.2) (layer "F.Cu") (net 17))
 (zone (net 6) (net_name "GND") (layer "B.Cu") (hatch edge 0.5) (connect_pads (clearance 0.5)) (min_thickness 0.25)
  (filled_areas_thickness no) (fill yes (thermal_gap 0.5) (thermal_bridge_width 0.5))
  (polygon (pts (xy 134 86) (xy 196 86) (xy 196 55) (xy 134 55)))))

